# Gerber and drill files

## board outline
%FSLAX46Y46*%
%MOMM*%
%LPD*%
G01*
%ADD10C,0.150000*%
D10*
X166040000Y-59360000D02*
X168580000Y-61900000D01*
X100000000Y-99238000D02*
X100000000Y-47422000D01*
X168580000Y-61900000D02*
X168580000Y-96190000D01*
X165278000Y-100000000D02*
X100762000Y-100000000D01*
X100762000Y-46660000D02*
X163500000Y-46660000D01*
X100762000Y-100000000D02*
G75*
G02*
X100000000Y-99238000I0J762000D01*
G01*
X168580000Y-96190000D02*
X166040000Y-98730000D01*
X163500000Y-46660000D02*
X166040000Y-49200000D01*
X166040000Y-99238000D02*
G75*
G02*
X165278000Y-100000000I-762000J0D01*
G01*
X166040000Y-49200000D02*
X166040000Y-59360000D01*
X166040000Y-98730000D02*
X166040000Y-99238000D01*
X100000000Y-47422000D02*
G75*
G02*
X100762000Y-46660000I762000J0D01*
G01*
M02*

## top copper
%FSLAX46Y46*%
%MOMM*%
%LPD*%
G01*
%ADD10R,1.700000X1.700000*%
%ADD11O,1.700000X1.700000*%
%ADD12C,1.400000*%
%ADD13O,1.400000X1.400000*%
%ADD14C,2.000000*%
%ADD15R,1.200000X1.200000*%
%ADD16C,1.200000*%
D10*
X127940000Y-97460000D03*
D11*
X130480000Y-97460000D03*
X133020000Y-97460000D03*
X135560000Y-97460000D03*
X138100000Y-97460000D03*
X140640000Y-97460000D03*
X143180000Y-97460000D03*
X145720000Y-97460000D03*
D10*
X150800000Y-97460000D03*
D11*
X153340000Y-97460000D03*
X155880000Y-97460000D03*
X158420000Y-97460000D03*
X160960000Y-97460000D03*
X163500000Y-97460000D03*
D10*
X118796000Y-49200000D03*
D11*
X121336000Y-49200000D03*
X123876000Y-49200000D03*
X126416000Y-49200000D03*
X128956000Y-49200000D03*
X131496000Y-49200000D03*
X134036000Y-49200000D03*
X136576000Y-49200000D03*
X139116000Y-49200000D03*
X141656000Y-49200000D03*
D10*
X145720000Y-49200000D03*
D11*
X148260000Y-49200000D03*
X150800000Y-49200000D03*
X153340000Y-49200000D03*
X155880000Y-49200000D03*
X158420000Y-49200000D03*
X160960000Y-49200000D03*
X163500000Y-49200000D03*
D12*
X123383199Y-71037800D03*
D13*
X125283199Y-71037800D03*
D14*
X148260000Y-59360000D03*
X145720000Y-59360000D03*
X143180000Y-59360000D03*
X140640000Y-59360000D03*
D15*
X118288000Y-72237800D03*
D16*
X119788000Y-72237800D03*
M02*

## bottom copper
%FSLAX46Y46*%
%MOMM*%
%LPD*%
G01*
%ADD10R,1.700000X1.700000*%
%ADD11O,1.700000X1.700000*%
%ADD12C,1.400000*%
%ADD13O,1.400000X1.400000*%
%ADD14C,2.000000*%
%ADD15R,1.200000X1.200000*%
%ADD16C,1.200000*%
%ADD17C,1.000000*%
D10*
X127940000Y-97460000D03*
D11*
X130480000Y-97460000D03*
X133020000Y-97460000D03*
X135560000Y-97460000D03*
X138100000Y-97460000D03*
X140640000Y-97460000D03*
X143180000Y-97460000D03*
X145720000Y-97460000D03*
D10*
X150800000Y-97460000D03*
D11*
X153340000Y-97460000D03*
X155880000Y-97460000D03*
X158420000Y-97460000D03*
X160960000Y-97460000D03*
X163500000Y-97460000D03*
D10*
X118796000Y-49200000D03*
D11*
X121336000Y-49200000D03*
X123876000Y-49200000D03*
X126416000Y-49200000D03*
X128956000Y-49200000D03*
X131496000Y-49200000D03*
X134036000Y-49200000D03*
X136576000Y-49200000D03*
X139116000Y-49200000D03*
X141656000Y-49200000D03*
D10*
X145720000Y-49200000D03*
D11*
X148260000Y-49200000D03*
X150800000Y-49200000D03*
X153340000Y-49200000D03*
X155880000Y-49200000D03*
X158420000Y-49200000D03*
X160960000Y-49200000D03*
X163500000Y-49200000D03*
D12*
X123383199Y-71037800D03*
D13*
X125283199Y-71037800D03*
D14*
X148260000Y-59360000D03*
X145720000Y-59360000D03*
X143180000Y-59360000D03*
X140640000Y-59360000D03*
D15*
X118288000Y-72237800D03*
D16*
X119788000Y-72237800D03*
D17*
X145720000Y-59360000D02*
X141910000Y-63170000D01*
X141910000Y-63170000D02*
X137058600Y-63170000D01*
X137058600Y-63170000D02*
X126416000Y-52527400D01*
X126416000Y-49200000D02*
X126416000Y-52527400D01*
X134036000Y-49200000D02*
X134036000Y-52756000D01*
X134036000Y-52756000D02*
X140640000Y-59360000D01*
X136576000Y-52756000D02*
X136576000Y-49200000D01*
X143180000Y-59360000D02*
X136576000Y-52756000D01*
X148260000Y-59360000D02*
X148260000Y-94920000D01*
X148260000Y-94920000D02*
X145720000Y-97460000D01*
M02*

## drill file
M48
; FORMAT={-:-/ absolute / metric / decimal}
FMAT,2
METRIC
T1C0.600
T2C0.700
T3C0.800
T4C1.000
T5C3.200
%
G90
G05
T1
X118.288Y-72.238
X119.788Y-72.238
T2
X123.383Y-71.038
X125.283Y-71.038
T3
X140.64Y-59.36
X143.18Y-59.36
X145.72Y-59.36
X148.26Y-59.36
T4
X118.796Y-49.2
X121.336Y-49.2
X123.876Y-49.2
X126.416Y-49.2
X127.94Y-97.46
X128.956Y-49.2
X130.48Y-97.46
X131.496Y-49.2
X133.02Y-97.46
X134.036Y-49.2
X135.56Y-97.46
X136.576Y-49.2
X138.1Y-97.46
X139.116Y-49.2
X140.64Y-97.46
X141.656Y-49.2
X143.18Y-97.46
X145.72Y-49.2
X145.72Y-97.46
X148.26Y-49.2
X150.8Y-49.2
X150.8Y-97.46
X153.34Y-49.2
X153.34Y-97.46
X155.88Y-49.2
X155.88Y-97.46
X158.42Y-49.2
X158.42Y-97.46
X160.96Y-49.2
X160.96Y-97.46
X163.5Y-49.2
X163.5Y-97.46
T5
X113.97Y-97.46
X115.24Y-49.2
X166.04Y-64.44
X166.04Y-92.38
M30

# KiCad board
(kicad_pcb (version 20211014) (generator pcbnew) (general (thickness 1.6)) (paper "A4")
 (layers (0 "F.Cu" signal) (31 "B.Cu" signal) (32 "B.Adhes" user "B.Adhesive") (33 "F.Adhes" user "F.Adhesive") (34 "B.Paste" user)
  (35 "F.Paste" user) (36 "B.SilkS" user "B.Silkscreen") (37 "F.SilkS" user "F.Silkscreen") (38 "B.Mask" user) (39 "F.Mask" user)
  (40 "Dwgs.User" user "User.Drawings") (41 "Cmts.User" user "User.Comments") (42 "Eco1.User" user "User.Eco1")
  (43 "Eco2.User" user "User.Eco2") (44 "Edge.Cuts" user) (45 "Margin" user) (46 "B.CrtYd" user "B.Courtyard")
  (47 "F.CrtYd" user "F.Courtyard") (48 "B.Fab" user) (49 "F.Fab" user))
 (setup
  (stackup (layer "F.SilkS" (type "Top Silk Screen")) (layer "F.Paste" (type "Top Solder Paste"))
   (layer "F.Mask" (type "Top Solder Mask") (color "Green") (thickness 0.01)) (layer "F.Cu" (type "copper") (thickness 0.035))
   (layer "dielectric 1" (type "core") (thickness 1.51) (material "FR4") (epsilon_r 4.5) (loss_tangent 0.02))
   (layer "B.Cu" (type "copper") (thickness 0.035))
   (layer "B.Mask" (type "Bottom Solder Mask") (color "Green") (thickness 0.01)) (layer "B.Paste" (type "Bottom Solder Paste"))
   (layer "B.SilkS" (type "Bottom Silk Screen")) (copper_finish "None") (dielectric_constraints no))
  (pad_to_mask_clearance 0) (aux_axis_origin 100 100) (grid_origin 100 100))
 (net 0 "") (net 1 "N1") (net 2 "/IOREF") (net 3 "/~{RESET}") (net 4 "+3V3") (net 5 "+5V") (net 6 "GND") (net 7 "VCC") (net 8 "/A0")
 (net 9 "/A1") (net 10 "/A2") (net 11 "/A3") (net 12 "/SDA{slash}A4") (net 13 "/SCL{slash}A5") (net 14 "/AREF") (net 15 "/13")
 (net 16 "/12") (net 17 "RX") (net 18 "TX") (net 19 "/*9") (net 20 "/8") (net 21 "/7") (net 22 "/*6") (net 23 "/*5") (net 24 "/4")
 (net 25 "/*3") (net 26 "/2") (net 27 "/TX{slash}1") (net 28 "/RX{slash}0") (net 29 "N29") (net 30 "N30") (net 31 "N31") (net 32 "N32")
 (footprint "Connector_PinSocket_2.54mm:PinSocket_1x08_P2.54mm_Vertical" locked (layer "F.Cu") (at 127.94 97.46 90)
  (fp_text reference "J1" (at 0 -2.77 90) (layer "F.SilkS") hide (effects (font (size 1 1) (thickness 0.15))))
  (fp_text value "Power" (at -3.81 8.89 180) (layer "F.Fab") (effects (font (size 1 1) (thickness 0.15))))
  (pad "1" thru_hole rect locked (at 0 0 90) (size 1.7 1.7) (drill 1) (layers *.Cu *.Mask) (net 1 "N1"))
  (pad "2" thru_hole oval locked (at 0 2.54 90) (size 1.7 1.7) (drill 1) (layers *.Cu *.Mask) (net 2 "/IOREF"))
  (pad "3" thru_hole oval locked (at 0 5.08 90) (size 1.7 1.7) (drill 1) (layers *.Cu *.Mask) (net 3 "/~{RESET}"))
  (pad "4" thru_hole oval locked (at 0 7.62 90) (size 1.7 1.7) (drill 1) (layers *.Cu *.Mask) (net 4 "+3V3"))
  (pad "5" thru_hole oval locked (at 0 10.16 90) (size 1.7 1.7) (drill 1) (layers *.Cu *.Mask) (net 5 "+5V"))
  (pad "6" thru_hole oval locked (at 0 12.7 90) (size 1.7 1.7) (drill 1) (layers *.Cu *.Mask) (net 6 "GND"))
  (pad "7" thru_hole oval locked (at 0 15.24 90) (size 1.7 1.7) (drill 1) (layers *.Cu *.Mask) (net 6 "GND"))
  (pad "8" thru_hole oval locked (at 0 17.78 90) (size 1.7 1.7) (drill 1) (layers *.Cu *.Mask) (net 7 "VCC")))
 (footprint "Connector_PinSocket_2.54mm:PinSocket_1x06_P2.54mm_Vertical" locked (layer "F.Cu") (at 150.8 97.46 90)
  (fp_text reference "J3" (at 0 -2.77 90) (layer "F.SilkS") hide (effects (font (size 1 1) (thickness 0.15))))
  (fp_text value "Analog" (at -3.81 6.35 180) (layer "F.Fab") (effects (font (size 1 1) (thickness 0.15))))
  (pad "1" thru_hole rect locked (at 0 0 90) (size 1.7 1.7) (drill 1) (layers *.Cu *.Mask) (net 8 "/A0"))
  (pad "2" thru_hole oval locked (at 0 2.54 90) (size 1.7 1.7) (drill 1) (layers *.Cu *.Mask) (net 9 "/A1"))
  (pad "3" thru_hole oval locked (at 0 5.08 90) (size 1.7 1.7) (drill 1) (layers *.Cu *.Mask) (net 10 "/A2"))
  (pad "4" thru_hole oval locked (at 0 7.62 90) (size 1.7 1.7) (drill 1) (layers *.Cu *.Mask) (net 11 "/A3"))
  (pad "5" thru_hole oval locked (at 0 10.16 90) (size 1.7 1.7) (drill 1) (layers *.Cu *.Mask) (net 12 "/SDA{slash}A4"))
  (pad "6" thru_hole oval locked (at 0 12.7 90) (size 1.7 1.7) (drill 1) (layers *.Cu *.Mask) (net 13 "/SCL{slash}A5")))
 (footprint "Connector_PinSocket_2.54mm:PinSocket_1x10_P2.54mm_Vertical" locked (layer "F.Cu") (at 118.796 49.2 90)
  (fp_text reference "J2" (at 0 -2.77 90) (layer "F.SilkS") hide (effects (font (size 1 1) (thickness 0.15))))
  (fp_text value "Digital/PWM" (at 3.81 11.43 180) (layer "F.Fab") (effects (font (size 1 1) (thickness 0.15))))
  (pad "1" thru_hole rect locked (at 0 0 90) (size 1.7 1.7) (drill 1) (layers *.Cu *.Mask) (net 13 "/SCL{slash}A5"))
  (pad "2" thru_hole oval locked (at 0 2.54 90) (size 1.7 1.7) (drill 1) (layers *.Cu *.Mask) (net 12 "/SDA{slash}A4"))
  (pad "3" thru_hole oval locked (at 0 5.08 90) (size 1.7 1.7) (drill 1) (layers *.Cu *.Mask) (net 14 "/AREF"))
  (pad "4" thru_hole oval locked (at 0 7.62 90) (size 1.7 1.7) (drill 1) (layers *.Cu *.Mask) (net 6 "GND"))
  (pad "5" thru_hole oval locked (at 0 10.16 90) (size 1.7 1.7) (drill 1) (layers *.Cu *.Mask) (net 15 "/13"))
  (pad "6" thru_hole oval locked (at 0 12.7 90) (size 1.7 1.7) (drill 1) (layers *.Cu *.Mask) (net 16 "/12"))
  (pad "7" thru_hole oval locked (at 0 15.24 90) (size 1.7 1.7) (drill 1) (layers *.Cu *.Mask) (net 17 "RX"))
  (pad "8" thru_hole oval locked (at 0 17.78 90) (size 1.7 1.7) (drill 1) (layers *.Cu *.Mask) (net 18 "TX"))
  (pad "9" thru_hole oval locked (at 0 20.32 90) (size 1.7 1.7) (drill 1) (layers *.Cu *.Mask) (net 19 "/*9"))
  (pad "10" thru_hole oval locked (at 0 22.86 90) (size 1.7 1.7) (drill 1) (layers *.Cu *.Mask) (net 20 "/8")))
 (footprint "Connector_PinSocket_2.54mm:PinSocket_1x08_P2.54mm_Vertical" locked (layer "F.Cu") (at 145.72 49.2 90)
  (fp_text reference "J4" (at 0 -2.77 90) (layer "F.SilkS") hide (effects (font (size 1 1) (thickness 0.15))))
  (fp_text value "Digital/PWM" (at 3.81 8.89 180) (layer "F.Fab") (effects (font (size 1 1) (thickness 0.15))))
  (pad "1" thru_hole rect locked (at 0 0 90) (size 1.7 1.7) (drill 1) (layers *.Cu *.Mask) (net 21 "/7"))
  (pad "2" thru_hole oval locked (at 0 2.54 90) (size 1.7 1.7) (drill 1) (layers *.Cu *.Mask) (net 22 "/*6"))
  (pad "3" thru_hole oval locked (at 0 5.08 90) (size 1.7 1.7) (drill 1) (layers *.Cu *.Mask) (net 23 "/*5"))
  (pad "4" thru_hole oval locked (at 0 7.62 90) (size 1.7 1.7) (drill 1) (layers *.Cu *.Mask) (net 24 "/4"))
  (pad "5" thru_hole oval locked (at 0 10.16 90) (size 1.7 1.7) (drill 1) (layers *.Cu *.Mask) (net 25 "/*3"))
  (pad "6" thru_hole oval locked (at 0 12.7 90) (size 1.7 1.7) (drill 1) (layers *.Cu *.Mask) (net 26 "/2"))
  (pad "7" thru_hole oval locked (at 0 15.24 90) (size 1.7 1.7) (drill 1) (layers *.Cu *.Mask) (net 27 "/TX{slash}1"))
  (pad "8" thru_hole oval locked (at 0 17.78 90) (size 1.7 1.7) (drill 1) (layers *.Cu *.Mask) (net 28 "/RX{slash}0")))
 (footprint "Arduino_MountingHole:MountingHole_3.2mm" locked (layer "F.Cu") (at 115.24 49.2)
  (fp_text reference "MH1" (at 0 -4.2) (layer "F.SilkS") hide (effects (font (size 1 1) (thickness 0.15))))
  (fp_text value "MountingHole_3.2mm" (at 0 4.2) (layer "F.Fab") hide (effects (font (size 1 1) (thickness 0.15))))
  (pad "" np_thru_hole circle locked (at 0 0) (size 3.2 3.2) (drill 3.2) (layers *.Cu *.Mask)))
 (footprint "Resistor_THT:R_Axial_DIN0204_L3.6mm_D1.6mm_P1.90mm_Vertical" (layer "F.Cu") (at 123.383199 71.0378)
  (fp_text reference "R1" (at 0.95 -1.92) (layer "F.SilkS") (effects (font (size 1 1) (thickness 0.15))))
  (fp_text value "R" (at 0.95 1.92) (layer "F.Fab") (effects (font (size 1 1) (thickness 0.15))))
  (pad "1" thru_hole circle (at 0 0) (size 1.4 1.4) (drill 0.7) (layers *.Cu *.Mask) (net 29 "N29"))
  (pad "2" thru_hole oval (at 1.9 0) (size 1.4 1.4) (drill 0.7) (layers *.Cu *.Mask) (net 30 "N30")))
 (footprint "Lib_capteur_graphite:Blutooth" (layer "F.Cu") (at 143.18 59.36 180)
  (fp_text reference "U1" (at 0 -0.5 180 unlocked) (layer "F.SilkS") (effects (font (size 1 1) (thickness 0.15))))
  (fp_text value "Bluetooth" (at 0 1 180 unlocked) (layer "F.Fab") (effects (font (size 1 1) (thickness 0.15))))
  (pad "1" thru_hole circle (at -5.08 0 180) (size 2 2) (drill 0.8) (layers *.Cu *.Mask) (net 7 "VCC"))
  (pad "2" thru_hole circle (at -2.54 0 180) (size 2 2) (drill 0.8) (layers *.Cu *.Mask) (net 6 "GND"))
  (pad "3" thru_hole circle (at 0 0 180) (size 2 2) (drill 0.8) (layers *.Cu *.Mask) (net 18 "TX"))
  (pad "4" thru_hole circle (at 2.54 0 180) (size 2 2) (drill 0.8) (layers *.Cu *.Mask) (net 17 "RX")))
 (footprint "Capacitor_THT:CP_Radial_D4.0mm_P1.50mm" (layer "F.Cu") (at 118.288 72.2378)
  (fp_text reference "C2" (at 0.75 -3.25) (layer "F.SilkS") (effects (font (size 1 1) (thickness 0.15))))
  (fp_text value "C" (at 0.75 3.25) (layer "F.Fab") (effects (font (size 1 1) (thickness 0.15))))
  (pad "1" thru_hole rect (at 0 0) (size 1.2 1.2) (drill 0.6) (layers *.Cu *.Mask) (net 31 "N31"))
  (pad "2" thru_hole circle (at 1.5 0) (size 1.2 1.2) (drill 0.6) (layers *.Cu *.Mask) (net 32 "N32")))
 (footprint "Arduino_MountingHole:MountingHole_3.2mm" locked (layer "F.Cu") (at 113.97 97.46)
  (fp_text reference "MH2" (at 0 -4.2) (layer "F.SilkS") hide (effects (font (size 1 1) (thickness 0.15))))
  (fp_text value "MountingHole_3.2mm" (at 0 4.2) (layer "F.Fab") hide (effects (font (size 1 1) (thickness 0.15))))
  (pad "" np_thru_hole circle locked (at 0 0) (size 3.2 3.2) (drill 3.2) (layers *.Cu *.Mask)))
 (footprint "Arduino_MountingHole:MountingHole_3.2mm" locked (layer "F.Cu") (at 166.04 64.44)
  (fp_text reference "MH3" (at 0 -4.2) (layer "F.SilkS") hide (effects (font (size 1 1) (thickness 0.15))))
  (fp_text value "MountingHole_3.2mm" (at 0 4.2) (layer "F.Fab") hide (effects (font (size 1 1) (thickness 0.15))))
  (pad "" np_thru_hole circle locked (at 0 0) (size 3.2 3.2) (drill 3.2) (layers *.Cu *.Mask)))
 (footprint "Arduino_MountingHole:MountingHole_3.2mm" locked (layer "F.Cu") (at 166.04 92.38)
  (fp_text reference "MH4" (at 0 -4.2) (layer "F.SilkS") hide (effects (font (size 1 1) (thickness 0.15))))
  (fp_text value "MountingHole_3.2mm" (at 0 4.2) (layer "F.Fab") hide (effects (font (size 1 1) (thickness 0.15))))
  (pad "" np_thru_hole circle locked (at 0 0) (size 3.2 3.2) (drill 3.2) (layers *.Cu *.Mask)))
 (gr_line (start 166.04 59.36) (end 168.58 61.9) (layer "Edge.Cuts") (width 0.15))
 (gr_line (start 100 99.238) (end 100 47.422) (layer "Edge.Cuts") (width 0.15))
 (gr_line (start 168.58 61.9) (end 168.58 96.19) (layer "Edge.Cuts") (width 0.15))
 (gr_line (start 165.278 100) (end 100.762 100) (layer "Edge.Cuts") (width 0.15))
 (gr_line (start 100.762 46.66) (end 163.5 46.66) (layer "Edge.Cuts") (width 0.15))
 (gr_arc (start 100.762 100) (mid 100.223185 99.776815) (end 100 99.238) (layer "Edge.Cuts") (width 0.15))
 (gr_line (start 168.58 96.19) (end 166.04 98.73) (layer "Edge.Cuts") (width 0.15))
 (gr_line (start 163.5 46.66) (end 166.04 49.2) (layer "Edge.Cuts") (width 0.15))
 (gr_arc (start 166.04 99.238) (mid 165.816815 99.776815) (end 165.278 100) (layer "Edge.Cuts") (width 0.15))
 (gr_line (start 166.04 49.2) (end 166.04 59.36) (layer "Edge.Cuts") (width 0.15))
 (gr_line (start 166.04 98.73) (end 166.04 99.238) (layer "Edge.Cuts") (width 0.15))
 (gr_arc (start 100 47.422) (mid 100.223185 46.883185) (end 100.762 46.66) (layer "Edge.Cuts") (width 0.15))
 (segment (start 145.72 59.36) (end 141.91 63.17) (width 1) (layer "B.Cu") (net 6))
 (segment (start 141.91 63.17) (end 137.0586 63.17) (width 1) (layer "B.Cu") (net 6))
 (segment (start 137.0586 63.17) (end 126.416 52.5274) (width 1) (layer "B.Cu") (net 6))
 (segment (start 126.416 49.2) (end 126.416 52.5274) (width 1) (layer "B.Cu") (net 6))
 (segment (start 134.036 49.2) (end 134.036 52.756) (width 1) (layer "B.Cu") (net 17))
 (segment (start 134.036 52.756) (end 140.64 59.36) (width 1) (layer "B.Cu") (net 17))
 (segment (start 136.576 52.756) (end 136.576 49.2) (width 1) (layer "B.Cu") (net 18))
 (segment (start 143.18 59.36) (end 136.576 52.756) (width 1) (layer "B.Cu") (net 18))
 (segment (start 148.26 59.36) (end 148.26 94.92) (width 1) (layer "B.Cu") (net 7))
 (segment (start 148.26 94.92) (end 145.72 97.46) (width 1) (layer "B.Cu") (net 7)))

